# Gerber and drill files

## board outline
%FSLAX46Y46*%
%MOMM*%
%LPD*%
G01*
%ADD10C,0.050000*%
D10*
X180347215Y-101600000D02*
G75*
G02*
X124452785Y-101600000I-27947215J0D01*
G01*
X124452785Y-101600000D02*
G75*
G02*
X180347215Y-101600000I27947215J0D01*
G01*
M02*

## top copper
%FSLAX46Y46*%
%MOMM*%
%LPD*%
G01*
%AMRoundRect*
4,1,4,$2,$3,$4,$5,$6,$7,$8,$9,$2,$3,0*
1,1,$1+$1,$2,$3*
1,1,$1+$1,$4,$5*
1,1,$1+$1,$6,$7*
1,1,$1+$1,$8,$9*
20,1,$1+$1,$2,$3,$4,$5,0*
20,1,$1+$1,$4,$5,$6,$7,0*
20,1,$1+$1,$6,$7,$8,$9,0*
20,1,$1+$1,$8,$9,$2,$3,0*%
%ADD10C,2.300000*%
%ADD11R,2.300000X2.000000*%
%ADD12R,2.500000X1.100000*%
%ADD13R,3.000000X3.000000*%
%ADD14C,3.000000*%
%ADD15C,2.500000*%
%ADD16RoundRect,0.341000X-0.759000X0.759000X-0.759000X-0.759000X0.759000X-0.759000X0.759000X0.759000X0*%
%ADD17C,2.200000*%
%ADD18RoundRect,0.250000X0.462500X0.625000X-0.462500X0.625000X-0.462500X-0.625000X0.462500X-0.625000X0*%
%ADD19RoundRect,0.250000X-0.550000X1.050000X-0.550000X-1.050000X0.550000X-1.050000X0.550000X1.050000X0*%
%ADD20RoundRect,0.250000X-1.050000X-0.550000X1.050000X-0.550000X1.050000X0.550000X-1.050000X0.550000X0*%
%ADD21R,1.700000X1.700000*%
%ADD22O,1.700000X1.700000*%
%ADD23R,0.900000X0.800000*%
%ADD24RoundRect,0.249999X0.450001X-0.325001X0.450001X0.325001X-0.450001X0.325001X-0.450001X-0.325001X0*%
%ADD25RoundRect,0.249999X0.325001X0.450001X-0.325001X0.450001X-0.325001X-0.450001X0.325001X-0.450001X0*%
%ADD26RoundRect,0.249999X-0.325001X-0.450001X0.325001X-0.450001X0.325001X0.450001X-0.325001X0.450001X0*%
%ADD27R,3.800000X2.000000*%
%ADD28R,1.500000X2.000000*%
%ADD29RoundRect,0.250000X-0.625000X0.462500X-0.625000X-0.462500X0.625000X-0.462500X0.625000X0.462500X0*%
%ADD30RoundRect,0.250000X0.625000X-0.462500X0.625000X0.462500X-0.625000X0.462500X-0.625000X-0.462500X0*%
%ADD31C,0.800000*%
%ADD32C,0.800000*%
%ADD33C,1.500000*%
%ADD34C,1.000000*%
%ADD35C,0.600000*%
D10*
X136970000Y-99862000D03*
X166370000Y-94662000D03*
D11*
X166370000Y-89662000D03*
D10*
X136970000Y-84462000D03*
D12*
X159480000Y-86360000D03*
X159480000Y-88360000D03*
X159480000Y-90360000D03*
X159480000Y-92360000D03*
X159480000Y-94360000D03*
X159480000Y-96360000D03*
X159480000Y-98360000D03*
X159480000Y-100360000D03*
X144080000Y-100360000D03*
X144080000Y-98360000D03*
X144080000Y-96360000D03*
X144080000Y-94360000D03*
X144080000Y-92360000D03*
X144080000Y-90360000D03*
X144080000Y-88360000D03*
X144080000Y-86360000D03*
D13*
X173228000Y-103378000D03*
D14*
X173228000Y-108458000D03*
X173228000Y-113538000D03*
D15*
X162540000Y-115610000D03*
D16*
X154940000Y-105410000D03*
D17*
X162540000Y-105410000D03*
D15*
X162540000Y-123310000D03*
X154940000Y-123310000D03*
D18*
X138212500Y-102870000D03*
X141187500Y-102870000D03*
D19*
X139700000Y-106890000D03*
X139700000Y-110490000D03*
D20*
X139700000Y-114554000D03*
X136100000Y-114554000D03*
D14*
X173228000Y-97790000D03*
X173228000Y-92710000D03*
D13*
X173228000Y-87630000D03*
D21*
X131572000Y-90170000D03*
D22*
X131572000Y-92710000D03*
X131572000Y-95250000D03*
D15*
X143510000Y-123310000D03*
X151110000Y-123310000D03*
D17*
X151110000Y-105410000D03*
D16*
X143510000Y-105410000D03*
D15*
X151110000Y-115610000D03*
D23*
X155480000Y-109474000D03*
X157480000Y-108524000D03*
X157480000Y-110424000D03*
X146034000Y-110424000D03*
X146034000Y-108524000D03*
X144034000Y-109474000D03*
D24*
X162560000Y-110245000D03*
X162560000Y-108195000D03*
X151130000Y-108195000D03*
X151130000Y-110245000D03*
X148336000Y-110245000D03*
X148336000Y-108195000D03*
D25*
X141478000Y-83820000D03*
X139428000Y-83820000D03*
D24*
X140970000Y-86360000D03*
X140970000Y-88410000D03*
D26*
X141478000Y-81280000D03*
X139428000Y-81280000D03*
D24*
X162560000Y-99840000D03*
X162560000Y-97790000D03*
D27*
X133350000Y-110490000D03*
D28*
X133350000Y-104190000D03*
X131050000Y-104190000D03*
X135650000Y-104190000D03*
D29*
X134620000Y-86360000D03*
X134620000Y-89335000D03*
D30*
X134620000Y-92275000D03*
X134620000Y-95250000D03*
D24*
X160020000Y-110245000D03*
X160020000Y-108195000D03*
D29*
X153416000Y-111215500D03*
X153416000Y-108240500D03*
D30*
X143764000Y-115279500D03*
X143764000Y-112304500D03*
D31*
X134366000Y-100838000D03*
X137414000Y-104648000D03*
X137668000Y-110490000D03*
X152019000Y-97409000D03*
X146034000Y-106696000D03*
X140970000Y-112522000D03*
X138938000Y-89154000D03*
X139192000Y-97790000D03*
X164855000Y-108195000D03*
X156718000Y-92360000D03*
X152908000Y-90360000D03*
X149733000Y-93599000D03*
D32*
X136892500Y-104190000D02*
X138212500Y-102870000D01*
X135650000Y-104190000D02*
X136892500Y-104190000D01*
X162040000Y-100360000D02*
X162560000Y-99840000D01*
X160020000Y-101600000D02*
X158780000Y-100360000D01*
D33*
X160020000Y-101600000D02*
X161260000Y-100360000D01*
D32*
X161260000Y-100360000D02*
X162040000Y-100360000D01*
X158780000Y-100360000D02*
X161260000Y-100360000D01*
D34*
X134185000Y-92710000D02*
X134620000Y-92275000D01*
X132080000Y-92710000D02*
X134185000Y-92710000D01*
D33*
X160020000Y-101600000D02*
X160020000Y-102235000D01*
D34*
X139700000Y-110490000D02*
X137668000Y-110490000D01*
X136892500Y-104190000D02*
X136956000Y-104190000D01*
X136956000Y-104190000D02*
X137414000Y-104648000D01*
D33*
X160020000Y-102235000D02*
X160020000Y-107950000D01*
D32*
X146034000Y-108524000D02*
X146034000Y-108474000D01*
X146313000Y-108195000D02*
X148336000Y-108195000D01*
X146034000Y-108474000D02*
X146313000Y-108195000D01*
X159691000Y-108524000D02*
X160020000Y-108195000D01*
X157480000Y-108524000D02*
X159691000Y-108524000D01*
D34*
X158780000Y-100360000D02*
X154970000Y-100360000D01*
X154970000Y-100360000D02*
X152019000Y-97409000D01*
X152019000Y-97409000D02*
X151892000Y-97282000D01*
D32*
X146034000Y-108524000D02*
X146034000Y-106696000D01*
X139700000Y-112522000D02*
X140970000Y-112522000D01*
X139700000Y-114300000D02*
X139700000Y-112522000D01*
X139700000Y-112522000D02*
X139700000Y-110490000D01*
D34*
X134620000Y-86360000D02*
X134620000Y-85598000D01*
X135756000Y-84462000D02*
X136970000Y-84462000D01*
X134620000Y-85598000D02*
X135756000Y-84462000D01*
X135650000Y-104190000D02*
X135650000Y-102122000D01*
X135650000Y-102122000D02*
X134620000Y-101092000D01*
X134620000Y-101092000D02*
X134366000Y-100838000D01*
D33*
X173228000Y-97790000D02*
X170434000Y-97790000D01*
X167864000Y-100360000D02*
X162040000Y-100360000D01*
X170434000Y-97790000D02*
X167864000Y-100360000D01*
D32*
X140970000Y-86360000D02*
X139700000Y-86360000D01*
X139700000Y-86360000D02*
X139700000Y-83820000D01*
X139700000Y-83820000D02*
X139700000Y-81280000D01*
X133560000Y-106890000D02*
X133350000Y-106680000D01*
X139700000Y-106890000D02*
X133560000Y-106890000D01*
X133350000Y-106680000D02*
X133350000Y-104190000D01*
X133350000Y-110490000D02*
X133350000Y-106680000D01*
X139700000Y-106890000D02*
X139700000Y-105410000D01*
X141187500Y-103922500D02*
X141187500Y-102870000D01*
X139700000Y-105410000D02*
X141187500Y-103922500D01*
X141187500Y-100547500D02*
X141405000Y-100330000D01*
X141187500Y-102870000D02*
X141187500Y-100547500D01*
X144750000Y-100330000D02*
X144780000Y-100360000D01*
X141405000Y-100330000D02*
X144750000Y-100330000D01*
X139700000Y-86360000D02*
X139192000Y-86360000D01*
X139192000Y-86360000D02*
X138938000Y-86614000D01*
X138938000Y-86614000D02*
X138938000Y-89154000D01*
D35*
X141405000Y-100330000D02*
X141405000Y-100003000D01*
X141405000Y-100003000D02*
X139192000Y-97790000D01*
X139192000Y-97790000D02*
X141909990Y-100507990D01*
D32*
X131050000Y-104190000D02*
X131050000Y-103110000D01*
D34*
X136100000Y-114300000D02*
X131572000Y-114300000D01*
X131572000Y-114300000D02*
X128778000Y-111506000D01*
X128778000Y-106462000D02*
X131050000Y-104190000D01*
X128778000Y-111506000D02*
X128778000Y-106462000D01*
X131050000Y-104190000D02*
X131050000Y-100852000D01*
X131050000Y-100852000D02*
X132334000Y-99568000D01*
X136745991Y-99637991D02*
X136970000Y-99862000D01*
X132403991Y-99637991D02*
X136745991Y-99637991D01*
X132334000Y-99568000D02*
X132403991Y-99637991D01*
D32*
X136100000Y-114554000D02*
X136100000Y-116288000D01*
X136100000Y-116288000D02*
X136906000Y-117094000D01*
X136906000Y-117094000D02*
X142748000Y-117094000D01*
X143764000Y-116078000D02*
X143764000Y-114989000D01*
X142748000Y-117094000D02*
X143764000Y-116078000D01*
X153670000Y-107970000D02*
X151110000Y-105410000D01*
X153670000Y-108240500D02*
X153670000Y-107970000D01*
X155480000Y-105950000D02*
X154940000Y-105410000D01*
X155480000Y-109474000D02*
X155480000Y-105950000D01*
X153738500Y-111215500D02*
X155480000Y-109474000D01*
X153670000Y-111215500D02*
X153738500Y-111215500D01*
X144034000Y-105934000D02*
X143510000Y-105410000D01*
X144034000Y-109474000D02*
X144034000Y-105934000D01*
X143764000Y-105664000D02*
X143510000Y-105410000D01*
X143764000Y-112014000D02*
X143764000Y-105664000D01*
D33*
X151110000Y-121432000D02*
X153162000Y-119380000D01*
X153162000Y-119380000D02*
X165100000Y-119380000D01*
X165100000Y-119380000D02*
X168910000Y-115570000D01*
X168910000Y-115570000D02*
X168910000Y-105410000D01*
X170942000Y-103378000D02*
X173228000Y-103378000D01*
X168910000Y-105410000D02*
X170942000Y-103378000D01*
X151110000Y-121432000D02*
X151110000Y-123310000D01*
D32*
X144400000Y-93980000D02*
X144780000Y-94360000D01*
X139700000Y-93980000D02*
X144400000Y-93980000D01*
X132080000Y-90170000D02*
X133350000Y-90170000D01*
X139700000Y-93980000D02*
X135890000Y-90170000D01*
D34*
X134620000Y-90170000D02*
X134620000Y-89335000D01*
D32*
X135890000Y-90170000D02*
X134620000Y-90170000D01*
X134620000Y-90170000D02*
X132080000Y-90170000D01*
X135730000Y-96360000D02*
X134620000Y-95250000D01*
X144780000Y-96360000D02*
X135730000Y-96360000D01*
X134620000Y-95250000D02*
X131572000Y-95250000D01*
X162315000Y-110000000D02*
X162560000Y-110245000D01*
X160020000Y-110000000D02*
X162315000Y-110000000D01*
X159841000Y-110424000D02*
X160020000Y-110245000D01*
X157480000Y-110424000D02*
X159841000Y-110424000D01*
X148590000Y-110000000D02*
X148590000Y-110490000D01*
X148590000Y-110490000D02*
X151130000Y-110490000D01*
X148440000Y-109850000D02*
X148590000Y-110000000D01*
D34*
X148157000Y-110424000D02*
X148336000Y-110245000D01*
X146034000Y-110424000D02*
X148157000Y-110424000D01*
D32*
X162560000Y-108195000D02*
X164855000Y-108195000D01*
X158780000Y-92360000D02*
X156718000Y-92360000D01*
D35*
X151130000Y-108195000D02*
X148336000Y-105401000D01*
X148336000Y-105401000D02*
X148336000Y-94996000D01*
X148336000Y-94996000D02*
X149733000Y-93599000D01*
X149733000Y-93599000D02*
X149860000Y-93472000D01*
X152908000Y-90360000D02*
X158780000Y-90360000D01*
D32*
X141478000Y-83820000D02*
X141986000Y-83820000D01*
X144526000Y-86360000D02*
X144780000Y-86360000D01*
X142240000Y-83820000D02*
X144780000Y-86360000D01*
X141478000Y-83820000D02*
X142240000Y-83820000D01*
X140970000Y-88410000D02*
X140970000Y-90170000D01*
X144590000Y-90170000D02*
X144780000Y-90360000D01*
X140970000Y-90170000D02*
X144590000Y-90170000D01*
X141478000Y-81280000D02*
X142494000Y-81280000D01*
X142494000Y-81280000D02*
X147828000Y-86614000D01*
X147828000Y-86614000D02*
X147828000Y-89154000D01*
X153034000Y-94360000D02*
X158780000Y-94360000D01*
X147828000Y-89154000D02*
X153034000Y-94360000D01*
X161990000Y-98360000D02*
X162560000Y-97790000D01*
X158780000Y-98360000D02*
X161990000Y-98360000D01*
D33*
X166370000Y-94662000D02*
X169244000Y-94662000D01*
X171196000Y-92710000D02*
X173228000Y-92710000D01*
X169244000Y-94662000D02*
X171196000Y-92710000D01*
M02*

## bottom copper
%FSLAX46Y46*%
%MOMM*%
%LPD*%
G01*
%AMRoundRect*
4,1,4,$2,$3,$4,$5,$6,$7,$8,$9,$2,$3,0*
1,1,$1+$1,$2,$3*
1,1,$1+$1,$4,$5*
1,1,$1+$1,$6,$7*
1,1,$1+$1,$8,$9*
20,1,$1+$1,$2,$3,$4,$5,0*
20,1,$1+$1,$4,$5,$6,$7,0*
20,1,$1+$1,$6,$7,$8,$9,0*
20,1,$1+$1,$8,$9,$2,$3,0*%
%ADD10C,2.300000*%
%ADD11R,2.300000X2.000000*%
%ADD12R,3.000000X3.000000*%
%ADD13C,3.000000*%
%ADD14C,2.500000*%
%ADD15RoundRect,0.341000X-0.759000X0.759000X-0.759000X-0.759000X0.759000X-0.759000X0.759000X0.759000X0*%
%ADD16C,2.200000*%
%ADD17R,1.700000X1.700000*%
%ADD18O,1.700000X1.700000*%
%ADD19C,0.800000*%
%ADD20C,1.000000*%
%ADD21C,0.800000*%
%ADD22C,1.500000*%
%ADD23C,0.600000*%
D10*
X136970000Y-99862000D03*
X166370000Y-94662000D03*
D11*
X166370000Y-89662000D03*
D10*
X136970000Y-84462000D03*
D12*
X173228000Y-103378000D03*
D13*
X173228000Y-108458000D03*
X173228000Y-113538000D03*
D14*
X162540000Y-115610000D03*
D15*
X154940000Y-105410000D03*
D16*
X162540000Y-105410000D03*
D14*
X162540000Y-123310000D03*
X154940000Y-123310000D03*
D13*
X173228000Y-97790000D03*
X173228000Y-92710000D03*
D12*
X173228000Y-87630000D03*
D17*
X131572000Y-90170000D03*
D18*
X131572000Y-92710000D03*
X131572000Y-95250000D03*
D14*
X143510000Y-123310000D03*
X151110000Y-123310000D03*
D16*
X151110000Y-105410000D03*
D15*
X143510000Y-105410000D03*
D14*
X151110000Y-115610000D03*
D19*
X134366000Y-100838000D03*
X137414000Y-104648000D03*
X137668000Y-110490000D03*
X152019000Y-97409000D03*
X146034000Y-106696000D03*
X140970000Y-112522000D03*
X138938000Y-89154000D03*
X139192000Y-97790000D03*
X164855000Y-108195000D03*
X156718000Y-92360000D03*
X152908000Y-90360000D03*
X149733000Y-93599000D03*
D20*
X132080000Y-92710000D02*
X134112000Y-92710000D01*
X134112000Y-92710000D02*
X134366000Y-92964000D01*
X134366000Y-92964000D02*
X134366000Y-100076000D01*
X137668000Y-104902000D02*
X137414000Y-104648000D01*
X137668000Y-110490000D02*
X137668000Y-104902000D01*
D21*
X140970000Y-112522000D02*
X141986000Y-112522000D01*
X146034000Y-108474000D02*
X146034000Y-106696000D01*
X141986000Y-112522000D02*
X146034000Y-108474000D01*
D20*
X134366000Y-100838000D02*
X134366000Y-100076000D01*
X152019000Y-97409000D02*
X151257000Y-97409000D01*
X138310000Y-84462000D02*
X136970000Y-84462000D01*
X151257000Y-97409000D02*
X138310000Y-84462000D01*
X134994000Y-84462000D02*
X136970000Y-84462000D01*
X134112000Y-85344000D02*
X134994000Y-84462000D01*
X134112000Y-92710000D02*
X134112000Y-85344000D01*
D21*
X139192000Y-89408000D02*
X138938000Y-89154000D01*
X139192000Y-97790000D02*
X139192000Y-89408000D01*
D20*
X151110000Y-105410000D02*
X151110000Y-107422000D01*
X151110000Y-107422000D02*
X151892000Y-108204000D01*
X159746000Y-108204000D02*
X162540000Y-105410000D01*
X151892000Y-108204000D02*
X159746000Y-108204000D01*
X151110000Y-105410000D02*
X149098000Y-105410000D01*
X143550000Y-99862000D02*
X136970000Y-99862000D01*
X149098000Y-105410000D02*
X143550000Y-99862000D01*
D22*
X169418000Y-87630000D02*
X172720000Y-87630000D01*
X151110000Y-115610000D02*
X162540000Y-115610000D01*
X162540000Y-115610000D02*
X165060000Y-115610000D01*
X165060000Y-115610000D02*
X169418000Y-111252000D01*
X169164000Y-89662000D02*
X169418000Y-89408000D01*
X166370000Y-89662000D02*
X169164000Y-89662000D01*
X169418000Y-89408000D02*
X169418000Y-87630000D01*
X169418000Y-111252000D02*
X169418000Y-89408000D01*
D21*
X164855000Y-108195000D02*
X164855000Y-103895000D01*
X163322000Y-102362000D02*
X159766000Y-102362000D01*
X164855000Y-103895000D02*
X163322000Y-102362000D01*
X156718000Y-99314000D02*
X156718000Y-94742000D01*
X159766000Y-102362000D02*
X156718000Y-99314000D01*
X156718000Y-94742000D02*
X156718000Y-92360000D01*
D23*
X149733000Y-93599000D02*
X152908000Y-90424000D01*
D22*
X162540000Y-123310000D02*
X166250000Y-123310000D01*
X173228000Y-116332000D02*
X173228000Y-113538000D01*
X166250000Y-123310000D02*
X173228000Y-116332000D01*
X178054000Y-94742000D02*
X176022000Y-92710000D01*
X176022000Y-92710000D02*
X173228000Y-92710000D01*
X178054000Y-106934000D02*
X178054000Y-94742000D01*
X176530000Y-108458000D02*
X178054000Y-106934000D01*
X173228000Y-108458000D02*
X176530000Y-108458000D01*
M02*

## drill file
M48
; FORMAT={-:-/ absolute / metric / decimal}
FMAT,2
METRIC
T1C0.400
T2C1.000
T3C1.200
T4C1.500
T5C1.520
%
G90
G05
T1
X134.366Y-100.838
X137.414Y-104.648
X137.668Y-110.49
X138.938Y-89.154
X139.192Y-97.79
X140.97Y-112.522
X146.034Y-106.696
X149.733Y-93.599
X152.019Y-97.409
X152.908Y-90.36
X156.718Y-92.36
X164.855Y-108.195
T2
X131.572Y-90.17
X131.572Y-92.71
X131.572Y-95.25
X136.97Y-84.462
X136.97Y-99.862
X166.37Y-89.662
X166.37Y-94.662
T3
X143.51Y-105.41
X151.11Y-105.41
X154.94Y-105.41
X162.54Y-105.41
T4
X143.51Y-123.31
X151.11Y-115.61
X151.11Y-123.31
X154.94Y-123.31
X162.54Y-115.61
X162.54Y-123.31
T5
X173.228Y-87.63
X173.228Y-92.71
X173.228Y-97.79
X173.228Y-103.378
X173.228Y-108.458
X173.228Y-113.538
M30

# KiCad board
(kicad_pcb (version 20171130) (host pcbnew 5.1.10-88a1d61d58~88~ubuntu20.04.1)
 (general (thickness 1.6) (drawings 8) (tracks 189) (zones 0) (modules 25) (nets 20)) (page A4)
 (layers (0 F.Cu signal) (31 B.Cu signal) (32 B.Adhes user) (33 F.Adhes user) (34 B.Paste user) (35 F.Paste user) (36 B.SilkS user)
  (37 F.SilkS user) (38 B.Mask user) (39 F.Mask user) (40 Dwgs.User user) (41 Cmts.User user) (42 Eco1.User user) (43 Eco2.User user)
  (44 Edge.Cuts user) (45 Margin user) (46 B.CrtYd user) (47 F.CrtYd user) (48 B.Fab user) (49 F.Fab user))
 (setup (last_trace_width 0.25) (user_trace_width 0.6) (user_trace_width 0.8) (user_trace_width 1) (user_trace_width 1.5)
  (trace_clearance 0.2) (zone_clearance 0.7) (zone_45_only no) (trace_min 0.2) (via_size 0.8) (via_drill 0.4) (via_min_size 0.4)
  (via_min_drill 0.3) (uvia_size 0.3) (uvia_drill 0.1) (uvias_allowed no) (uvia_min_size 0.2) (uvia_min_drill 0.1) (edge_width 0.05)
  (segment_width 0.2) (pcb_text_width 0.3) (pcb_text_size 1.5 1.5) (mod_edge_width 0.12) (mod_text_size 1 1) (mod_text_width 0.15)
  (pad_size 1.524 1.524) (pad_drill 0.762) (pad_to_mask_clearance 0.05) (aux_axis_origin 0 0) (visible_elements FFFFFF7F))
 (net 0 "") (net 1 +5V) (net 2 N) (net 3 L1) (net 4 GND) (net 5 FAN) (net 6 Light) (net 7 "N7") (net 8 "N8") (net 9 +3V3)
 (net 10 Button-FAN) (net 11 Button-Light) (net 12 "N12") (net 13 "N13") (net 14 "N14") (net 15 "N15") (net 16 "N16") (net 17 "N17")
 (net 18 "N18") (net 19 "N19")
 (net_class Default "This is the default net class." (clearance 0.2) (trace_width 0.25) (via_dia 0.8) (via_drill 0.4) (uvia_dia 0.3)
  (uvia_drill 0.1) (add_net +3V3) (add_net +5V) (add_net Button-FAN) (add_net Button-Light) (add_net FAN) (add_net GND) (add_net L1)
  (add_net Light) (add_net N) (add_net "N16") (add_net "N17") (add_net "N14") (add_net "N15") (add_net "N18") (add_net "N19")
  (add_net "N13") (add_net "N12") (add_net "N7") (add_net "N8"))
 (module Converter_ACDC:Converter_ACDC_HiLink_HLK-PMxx (layer B.Cu) (at 166.37 89.662 180)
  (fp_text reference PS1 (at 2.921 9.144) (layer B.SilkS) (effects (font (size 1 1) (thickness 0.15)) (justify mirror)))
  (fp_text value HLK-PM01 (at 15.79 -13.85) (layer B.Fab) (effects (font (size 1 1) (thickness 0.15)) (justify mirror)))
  (pad 4 thru_hole circle (at 29.4 -10.2 180) (size 2.3 2.3) (drill 1) (layers *.Cu *.Mask) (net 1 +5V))
  (pad 2 thru_hole circle (at 0 -5 180) (size 2.3 2.3) (drill 1) (layers *.Cu *.Mask) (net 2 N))
  (pad 1 thru_hole rect (at 0 0 180) (size 2.3 2) (drill 1) (layers *.Cu *.Mask) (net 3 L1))
  (pad 3 thru_hole circle (at 29.4 5.2 180) (size 2.3 2.3) (drill 1) (layers *.Cu *.Mask) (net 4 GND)))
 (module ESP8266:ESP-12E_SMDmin (layer F.Cu) (at 144.78 86.36)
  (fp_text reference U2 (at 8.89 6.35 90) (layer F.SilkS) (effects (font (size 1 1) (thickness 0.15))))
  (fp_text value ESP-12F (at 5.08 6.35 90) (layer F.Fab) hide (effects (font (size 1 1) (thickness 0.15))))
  (pad 16 smd rect (at 14 0) (size 2.5 1.1) (drill (offset 0.7 0)) (layers F.Cu F.Paste F.Mask))
  (pad 15 smd rect (at 14 2) (size 2.5 1.1) (drill (offset 0.7 0)) (layers F.Cu F.Paste F.Mask))
  (pad 14 smd rect (at 14 4) (size 2.5 1.1) (drill (offset 0.7 0)) (layers F.Cu F.Paste F.Mask) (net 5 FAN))
  (pad 13 smd rect (at 14 6) (size 2.5 1.1) (drill (offset 0.7 0)) (layers F.Cu F.Paste F.Mask) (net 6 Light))
  (pad 12 smd rect (at 14 8) (size 2.5 1.1) (drill (offset 0.7 0)) (layers F.Cu F.Paste F.Mask) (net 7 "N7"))
  (pad 11 smd rect (at 14 10) (size 2.5 1.1) (drill (offset 0.7 0)) (layers F.Cu F.Paste F.Mask))
  (pad 10 smd rect (at 14 12) (size 2.5 1.1) (drill (offset 0.7 0)) (layers F.Cu F.Paste F.Mask) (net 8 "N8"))
  (pad 9 smd rect (at 14 14) (size 2.5 1.1) (drill (offset 0.7 0)) (layers F.Cu F.Paste F.Mask) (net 4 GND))
  (pad 8 smd rect (at 0 14) (size 2.5 1.1) (drill (offset -0.7 0)) (layers F.Cu F.Paste F.Mask) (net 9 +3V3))
  (pad 7 smd rect (at 0 12) (size 2.5 1.1) (drill (offset -0.7 0)) (layers F.Cu F.Paste F.Mask))
  (pad 6 smd rect (at 0 10) (size 2.5 1.1) (drill (offset -0.7 0)) (layers F.Cu F.Paste F.Mask) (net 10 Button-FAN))
  (pad 5 smd rect (at 0 8) (size 2.5 1.1) (drill (offset -0.7 0)) (layers F.Cu F.Paste F.Mask) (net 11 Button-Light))
  (pad 4 smd rect (at 0 6) (size 2.5 1.1) (drill (offset -0.7 0)) (layers F.Cu F.Paste F.Mask))
  (pad 3 smd rect (at 0 4) (size 2.5 1.1) (drill (offset -0.7 0)) (layers F.Cu F.Paste F.Mask) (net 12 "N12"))
  (pad 2 smd rect (at 0 2) (size 2.5 1.1) (drill (offset -0.7 0)) (layers F.Cu F.Paste F.Mask))
  (pad 1 smd rect (at 0 0) (size 2.5 1.1) (drill (offset -0.7 0)) (layers F.Cu F.Paste F.Mask) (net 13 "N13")))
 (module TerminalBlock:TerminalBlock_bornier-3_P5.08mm (layer B.Cu) (at 173.228 103.378 270)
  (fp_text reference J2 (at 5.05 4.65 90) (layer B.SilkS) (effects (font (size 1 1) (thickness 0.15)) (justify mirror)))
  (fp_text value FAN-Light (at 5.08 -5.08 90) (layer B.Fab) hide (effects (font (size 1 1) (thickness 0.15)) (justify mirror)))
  (pad 1 thru_hole rect (at 0 0 270) (size 3 3) (drill 1.52) (layers *.Cu *.Mask) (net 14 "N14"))
  (pad 2 thru_hole circle (at 5.08 0 270) (size 3 3) (drill 1.52) (layers *.Cu *.Mask) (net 2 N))
  (pad 3 thru_hole circle (at 10.16 0 270) (size 3 3) (drill 1.52) (layers *.Cu *.Mask) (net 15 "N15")))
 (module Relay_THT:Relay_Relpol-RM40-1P (layer B.Cu) (at 154.94 105.41 270)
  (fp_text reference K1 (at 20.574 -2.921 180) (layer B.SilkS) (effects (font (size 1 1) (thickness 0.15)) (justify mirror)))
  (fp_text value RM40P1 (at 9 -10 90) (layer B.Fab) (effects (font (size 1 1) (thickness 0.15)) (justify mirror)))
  (pad 11 thru_hole circle (at 10.2 -7.6 270) (size 2.5 2.5) (drill 1.5) (layers *.Cu *.Mask) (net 3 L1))
  (pad A2 thru_hole roundrect (at 0 0 270) (size 2.2 2.2) (drill 1.2) (layers *.Cu *.Mask) (roundrect_rratio 0.155) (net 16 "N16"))
  (pad A1 thru_hole circle (at 0 -7.6 270) (size 2.2 2.2) (drill 1.2) (layers *.Cu *.Mask) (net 1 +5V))
  (pad 14 thru_hole circle (at 17.9 -7.6 270) (size 2.5 2.5) (drill 1.5) (layers *.Cu *.Mask) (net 15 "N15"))
  (pad 12 thru_hole circle (at 17.9 0 270) (size 2.5 2.5) (drill 1.5) (layers *.Cu *.Mask)))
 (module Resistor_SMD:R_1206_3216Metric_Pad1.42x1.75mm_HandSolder (layer F.Cu) (at 139.7 102.87 180)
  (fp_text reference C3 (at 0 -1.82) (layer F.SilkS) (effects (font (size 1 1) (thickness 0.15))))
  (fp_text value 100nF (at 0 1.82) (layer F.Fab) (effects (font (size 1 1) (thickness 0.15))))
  (pad 2 smd roundrect (at 1.4875 0 180) (size 1.425 1.75) (layers F.Cu F.Paste F.Mask) (roundrect_rratio 0.1754385964912281) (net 4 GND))
  (pad 1 smd roundrect (at -1.4875 0 180) (size 1.425 1.75) (layers F.Cu F.Paste F.Mask) (roundrect_rratio 0.1754385964912281) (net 9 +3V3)))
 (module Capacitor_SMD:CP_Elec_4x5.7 (layer F.Cu) (at 139.7 108.69 270)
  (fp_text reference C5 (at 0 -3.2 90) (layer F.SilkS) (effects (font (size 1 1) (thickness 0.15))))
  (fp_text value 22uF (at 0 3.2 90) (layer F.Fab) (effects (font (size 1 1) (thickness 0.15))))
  (pad 1 smd roundrect (at -1.8 0 270) (size 2.6 1.6) (layers F.Cu F.Paste F.Mask) (roundrect_rratio 0.15625) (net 9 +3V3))
  (pad 2 smd roundrect (at 1.8 0 270) (size 2.6 1.6) (layers F.Cu F.Paste F.Mask) (roundrect_rratio 0.15625) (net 4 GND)))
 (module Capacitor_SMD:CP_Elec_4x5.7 (layer F.Cu) (at 137.9 114.554)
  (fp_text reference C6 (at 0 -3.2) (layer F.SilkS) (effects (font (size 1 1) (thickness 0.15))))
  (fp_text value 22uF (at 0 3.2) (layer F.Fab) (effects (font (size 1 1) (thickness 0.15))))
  (pad 2 smd roundrect (at 1.8 0) (size 2.6 1.6) (layers F.Cu F.Paste F.Mask) (roundrect_rratio 0.15625) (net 4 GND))
  (pad 1 smd roundrect (at -1.8 0) (size 2.6 1.6) (layers F.Cu F.Paste F.Mask) (roundrect_rratio 0.15625) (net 1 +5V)))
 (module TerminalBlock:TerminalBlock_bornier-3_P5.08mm (layer B.Cu) (at 173.228 87.63 270)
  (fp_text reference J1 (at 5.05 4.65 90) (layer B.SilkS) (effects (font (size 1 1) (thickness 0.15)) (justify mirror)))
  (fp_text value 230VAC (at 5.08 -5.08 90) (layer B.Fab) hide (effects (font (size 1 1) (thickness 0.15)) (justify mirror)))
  (pad 3 thru_hole circle (at 10.16 0 270) (size 3 3) (drill 1.52) (layers *.Cu *.Mask) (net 4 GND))
  (pad 2 thru_hole circle (at 5.08 0 270) (size 3 3) (drill 1.52) (layers *.Cu *.Mask) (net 2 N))
  (pad 1 thru_hole rect (at 0 0 270) (size 3 3) (drill 1.52) (layers *.Cu *.Mask) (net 3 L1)))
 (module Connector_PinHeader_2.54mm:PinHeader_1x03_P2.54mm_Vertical (layer F.Cu) (at 131.572 90.17)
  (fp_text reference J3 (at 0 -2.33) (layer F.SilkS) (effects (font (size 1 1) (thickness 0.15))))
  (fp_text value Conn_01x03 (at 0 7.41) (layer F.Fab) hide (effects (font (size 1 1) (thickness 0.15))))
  (pad 1 thru_hole rect (at 0 0) (size 1.7 1.7) (drill 1) (layers *.Cu *.Mask) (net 11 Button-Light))
  (pad 2 thru_hole oval (at 0 2.54) (size 1.7 1.7) (drill 1) (layers *.Cu *.Mask) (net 4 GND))
  (pad 3 thru_hole oval (at 0 5.08) (size 1.7 1.7) (drill 1) (layers *.Cu *.Mask) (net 10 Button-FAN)))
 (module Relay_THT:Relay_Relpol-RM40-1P (layer B.Cu) (at 143.51 105.41 270)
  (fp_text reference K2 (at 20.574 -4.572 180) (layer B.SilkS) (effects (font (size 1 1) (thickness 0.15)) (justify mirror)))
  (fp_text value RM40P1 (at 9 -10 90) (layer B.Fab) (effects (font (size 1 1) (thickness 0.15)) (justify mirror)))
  (pad 12 thru_hole circle (at 17.9 0 270) (size 2.5 2.5) (drill 1.5) (layers *.Cu *.Mask))
  (pad 14 thru_hole circle (at 17.9 -7.6 270) (size 2.5 2.5) (drill 1.5) (layers *.Cu *.Mask) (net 14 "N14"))
  (pad A1 thru_hole circle (at 0 -7.6 270) (size 2.2 2.2) (drill 1.2) (layers *.Cu *.Mask) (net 1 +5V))
  (pad A2 thru_hole roundrect (at 0 0 270) (size 2.2 2.2) (drill 1.2) (layers *.Cu *.Mask) (roundrect_rratio 0.155) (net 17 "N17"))
  (pad 11 thru_hole circle (at 10.2 -7.6 270) (size 2.5 2.5) (drill 1.5) (layers *.Cu *.Mask) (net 3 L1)))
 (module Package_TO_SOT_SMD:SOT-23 (layer F.Cu) (at 156.48 109.474 180)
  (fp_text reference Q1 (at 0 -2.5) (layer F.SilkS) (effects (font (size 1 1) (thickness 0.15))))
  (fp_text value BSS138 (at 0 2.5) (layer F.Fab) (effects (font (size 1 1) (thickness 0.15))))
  (pad 3 smd rect (at 1 0 180) (size 0.9 0.8) (layers F.Cu F.Paste F.Mask) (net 16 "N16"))
  (pad 2 smd rect (at -1 0.95 180) (size 0.9 0.8) (layers F.Cu F.Paste F.Mask) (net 4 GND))
  (pad 1 smd rect (at -1 -0.95 180) (size 0.9 0.8) (layers F.Cu F.Paste F.Mask) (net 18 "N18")))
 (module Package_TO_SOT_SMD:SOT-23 (layer F.Cu) (at 145.034 109.474 180)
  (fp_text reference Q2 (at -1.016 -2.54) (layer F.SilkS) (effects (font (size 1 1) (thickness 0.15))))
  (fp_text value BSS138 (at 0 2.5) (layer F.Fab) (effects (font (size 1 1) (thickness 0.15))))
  (pad 1 smd rect (at -1 -0.95 180) (size 0.9 0.8) (layers F.Cu F.Paste F.Mask) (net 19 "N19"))
  (pad 2 smd rect (at -1 0.95 180) (size 0.9 0.8) (layers F.Cu F.Paste F.Mask) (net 4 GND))
  (pad 3 smd rect (at 1 0 180) (size 0.9 0.8) (layers F.Cu F.Paste F.Mask) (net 17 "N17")))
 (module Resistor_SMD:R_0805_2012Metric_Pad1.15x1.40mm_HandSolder (layer F.Cu) (at 162.56 109.22 90)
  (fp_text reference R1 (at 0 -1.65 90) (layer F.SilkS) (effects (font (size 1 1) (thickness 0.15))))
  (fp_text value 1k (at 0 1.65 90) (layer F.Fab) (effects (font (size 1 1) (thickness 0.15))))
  (pad 1 smd roundrect (at -1.025 0 90) (size 1.15 1.4) (layers F.Cu F.Paste F.Mask) (roundrect_rratio 0.2173904347826087) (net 18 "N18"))
  (pad 2 smd roundrect (at 1.025 0 90) (size 1.15 1.4) (layers F.Cu F.Paste F.Mask) (roundrect_rratio 0.2173904347826087) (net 6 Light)))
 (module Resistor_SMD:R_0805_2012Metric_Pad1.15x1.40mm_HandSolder (layer F.Cu) (at 151.13 109.22 90)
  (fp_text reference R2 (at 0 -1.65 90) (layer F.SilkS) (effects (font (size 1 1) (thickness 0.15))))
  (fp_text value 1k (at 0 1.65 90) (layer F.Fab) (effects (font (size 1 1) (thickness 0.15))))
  (pad 2 smd roundrect (at 1.025 0 90) (size 1.15 1.4) (layers F.Cu F.Paste F.Mask) (roundrect_rratio 0.2173904347826087) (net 5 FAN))
  (pad 1 smd roundrect (at -1.025 0 90) (size 1.15 1.4) (layers F.Cu F.Paste F.Mask) (roundrect_rratio 0.2173904347826087) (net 19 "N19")))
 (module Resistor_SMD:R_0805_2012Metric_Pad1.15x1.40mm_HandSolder (layer F.Cu) (at 148.336 109.22 90)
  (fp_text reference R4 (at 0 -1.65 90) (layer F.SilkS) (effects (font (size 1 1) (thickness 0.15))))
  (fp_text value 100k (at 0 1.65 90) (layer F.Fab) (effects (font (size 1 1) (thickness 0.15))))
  (pad 1 smd roundrect (at -1.025 0 90) (size 1.15 1.4) (layers F.Cu F.Paste F.Mask) (roundrect_rratio 0.2173904347826087) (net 19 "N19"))
  (pad 2 smd roundrect (at 1.025 0 90) (size 1.15 1.4) (layers F.Cu F.Paste F.Mask) (roundrect_rratio 0.2173904347826087) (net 4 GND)))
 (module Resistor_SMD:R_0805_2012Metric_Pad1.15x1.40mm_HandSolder (layer F.Cu) (at 140.453 83.82 180)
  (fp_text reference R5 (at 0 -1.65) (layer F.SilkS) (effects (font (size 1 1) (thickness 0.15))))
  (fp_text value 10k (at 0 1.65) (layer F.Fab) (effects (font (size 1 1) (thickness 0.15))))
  (pad 1 smd roundrect (at -1.025 0 180) (size 1.15 1.4) (layers F.Cu F.Paste F.Mask) (roundrect_rratio 0.2173904347826087) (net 13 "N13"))
  (pad 2 smd roundrect (at 1.025 0 180) (size 1.15 1.4) (layers F.Cu F.Paste F.Mask) (roundrect_rratio 0.2173904347826087) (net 9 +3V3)))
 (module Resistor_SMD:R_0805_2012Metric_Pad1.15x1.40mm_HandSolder (layer F.Cu) (at 140.97 87.385 90)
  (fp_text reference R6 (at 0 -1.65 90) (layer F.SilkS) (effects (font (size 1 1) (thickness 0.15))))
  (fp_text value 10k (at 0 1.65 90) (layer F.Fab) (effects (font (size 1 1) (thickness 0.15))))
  (pad 2 smd roundrect (at 1.025 0 90) (size 1.15 1.4) (layers F.Cu F.Paste F.Mask) (roundrect_rratio 0.2173904347826087) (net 9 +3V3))
  (pad 1 smd roundrect (at -1.025 0 90) (size 1.15 1.4) (layers F.Cu F.Paste F.Mask) (roundrect_rratio 0.2173904347826087) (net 12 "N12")))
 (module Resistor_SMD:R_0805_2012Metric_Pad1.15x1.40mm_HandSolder (layer F.Cu) (at 140.453 81.28)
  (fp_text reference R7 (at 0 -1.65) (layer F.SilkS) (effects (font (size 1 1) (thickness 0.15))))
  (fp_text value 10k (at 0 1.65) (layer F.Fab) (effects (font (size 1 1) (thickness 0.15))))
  (pad 2 smd roundrect (at 1.025 0) (size 1.15 1.4) (layers F.Cu F.Paste F.Mask) (roundrect_rratio 0.2173904347826087) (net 7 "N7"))
  (pad 1 smd roundrect (at -1.025 0) (size 1.15 1.4) (layers F.Cu F.Paste F.Mask) (roundrect_rratio 0.2173904347826087) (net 9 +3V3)))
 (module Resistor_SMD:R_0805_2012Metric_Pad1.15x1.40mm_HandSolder (layer F.Cu) (at 162.56 98.815 90)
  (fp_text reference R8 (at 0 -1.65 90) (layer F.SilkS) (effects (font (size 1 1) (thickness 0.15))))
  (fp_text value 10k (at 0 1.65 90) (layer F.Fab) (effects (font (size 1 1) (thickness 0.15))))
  (pad 1 smd roundrect (at -1.025 0 90) (size 1.15 1.4) (layers F.Cu F.Paste F.Mask) (roundrect_rratio 0.2173904347826087) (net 4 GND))
  (pad 2 smd roundrect (at 1.025 0 90) (size 1.15 1.4) (layers F.Cu F.Paste F.Mask) (roundrect_rratio 0.2173904347826087) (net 8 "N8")))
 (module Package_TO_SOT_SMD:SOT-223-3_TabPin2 (layer F.Cu) (at 133.35 107.34 270)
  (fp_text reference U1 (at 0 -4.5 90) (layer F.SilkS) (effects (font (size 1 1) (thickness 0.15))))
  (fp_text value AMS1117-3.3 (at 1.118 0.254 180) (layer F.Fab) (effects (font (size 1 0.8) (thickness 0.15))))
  (pad 2 smd rect (at 3.15 0 270) (size 2 3.8) (layers F.Cu F.Paste F.Mask) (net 9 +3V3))
  (pad 2 smd rect (at -3.15 0 270) (size 2 1.5) (layers F.Cu F.Paste F.Mask) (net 9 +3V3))
  (pad 3 smd rect (at -3.15 2.3 270) (size 2 1.5) (layers F.Cu F.Paste F.Mask) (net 1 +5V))
  (pad 1 smd rect (at -3.15 -2.3 270) (size 2 1.5) (layers F.Cu F.Paste F.Mask) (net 4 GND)))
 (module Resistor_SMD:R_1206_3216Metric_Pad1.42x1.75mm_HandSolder (layer F.Cu) (at 134.62 87.8475 270)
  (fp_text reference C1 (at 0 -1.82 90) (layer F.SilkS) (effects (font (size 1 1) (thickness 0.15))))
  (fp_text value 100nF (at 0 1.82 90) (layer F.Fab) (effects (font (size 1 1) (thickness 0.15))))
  (pad 1 smd roundrect (at -1.4875 0 270) (size 1.425 1.75) (layers F.Cu F.Paste F.Mask) (roundrect_rratio 0.1754385964912281) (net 4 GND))
  (pad 2 smd roundrect (at 1.4875 0 270) (size 1.425 1.75) (layers F.Cu F.Paste F.Mask) (roundrect_rratio 0.1754385964912281)
   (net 11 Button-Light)))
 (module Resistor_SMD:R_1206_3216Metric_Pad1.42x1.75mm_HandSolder (layer F.Cu) (at 134.62 93.7625 90)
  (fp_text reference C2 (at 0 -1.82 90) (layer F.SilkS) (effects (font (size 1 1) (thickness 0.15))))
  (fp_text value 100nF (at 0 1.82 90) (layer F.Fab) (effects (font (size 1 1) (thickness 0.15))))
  (pad 2 smd roundrect (at 1.4875 0 90) (size 1.425 1.75) (layers F.Cu F.Paste F.Mask) (roundrect_rratio 0.1754385964912281) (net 4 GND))
  (pad 1 smd roundrect (at -1.4875 0 90) (size 1.425 1.75) (layers F.Cu F.Paste F.Mask) (roundrect_rratio 0.1754385964912281)
   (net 10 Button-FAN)))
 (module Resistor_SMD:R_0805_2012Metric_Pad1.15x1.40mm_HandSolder (layer F.Cu) (at 160.02 109.22 90)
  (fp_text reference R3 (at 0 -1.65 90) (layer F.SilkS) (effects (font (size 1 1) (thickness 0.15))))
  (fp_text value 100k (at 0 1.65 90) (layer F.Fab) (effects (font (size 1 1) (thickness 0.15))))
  (pad 1 smd roundrect (at -1.025 0 90) (size 1.15 1.4) (layers F.Cu F.Paste F.Mask) (roundrect_rratio 0.2173904347826087) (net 18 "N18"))
  (pad 2 smd roundrect (at 1.025 0 90) (size 1.15 1.4) (layers F.Cu F.Paste F.Mask) (roundrect_rratio 0.2173904347826087) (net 4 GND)))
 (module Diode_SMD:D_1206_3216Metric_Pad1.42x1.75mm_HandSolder (layer F.Cu) (at 153.416 109.728 270)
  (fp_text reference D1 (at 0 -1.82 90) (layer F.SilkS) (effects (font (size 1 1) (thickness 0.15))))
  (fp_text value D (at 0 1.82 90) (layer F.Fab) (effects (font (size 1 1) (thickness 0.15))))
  (pad 2 smd roundrect (at 1.4875 0 270) (size 1.425 1.75) (layers F.Cu F.Paste F.Mask) (roundrect_rratio 0.1754385964912281) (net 16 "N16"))
  (pad 1 smd roundrect (at -1.4875 0 270) (size 1.425 1.75) (layers F.Cu F.Paste F.Mask) (roundrect_rratio 0.1754385964912281) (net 1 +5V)))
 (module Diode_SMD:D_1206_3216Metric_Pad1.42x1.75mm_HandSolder (layer F.Cu) (at 143.764 113.792 90)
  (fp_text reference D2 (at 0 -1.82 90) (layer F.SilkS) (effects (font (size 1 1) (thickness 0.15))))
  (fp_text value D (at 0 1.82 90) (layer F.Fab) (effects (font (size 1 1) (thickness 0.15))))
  (pad 1 smd roundrect (at -1.4875 0 90) (size 1.425 1.75) (layers F.Cu F.Paste F.Mask) (roundrect_rratio 0.1754385964912281) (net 1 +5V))
  (pad 2 smd roundrect (at 1.4875 0 90) (size 1.425 1.75) (layers F.Cu F.Paste F.Mask) (roundrect_rratio 0.1754385964912281) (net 17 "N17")))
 (gr_circle (center 152.4 101.6) (end 153.035 73.66) (layer Edge.Cuts) (width 0.05))
 (segment (start 136.8925 104.19) (end 138.2125 102.87) (width 0.8) (layer F.Cu) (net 4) (status 20))
 (segment (start 135.65 104.19) (end 136.8925 104.19) (width 0.8) (layer F.Cu) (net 4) (status 10))
 (segment (start 162.04 100.36) (end 162.56 99.84) (width 0.8) (layer F.Cu) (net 4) (status 30))
 (segment (start 160.02 101.6) (end 158.78 100.36) (width 0.8) (layer F.Cu) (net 4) (status 20))
 (segment (start 160.02 101.6) (end 161.26 100.36) (width 1.5) (layer F.Cu) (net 4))
 (segment (start 161.26 100.36) (end 162.04 100.36) (width 0.8) (layer F.Cu) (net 4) (status 20))
 (segment (start 158.78 100.36) (end 161.26 100.36) (width 0.8) (layer F.Cu) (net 4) (status 10))
 (segment (start 134.185 92.71) (end 134.62 92.275) (width 1) (layer F.Cu) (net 4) (status 30))
 (segment (start 132.08 92.71) (end 134.185 92.71) (width 1) (layer F.Cu) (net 4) (status 30))
 (segment (start 160.02 101.6) (end 160.02 102.235) (width 1.5) (layer F.Cu) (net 4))
 (segment (start 132.08 92.71) (end 134.112 92.71) (width 1) (layer B.Cu) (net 4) (status 10))
 (segment (start 134.112 92.71) (end 134.366 92.964) (width 1) (layer B.Cu) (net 4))
 (segment (start 134.366 92.964) (end 134.366 100.076) (width 1) (layer B.Cu) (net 4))
 (via (at 134.366 100.838) (size 0.8) (drill 0.4) (layers F.Cu B.Cu) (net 4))
 (segment (start 139.7 110.49) (end 137.668 110.49) (width 1) (layer F.Cu) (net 4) (status 10))
 (segment (start 136.8925 104.19) (end 136.956 104.19) (width 1) (layer F.Cu) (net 4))
 (segment (start 136.956 104.19) (end 137.414 104.648) (width 1) (layer F.Cu) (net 4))
 (via (at 137.414 104.648) (size 0.8) (drill 0.4) (layers F.Cu B.Cu) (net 4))
 (via (at 137.668 110.49) (size 0.8) (drill 0.4) (layers F.Cu B.Cu) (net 4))
 (segment (start 137.668 104.902) (end 137.414 104.648) (width 1) (layer B.Cu) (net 4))
 (segment (start 137.668 110.49) (end 137.668 104.902) (width 1) (layer B.Cu) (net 4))
 (segment (start 160.02 102.235) (end 160.02 107.95) (width 1.5) (layer F.Cu) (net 4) (status 20))
 (segment (start 146.034 108.524) (end 146.034 108.474) (width 0.8) (layer F.Cu) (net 4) (status 30))
 (segment (start 146.313 108.195) (end 148.336 108.195) (width 0.8) (layer F.Cu) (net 4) (status 30))
 (segment (start 146.034 108.474) (end 146.313 108.195) (width 0.8) (layer F.Cu) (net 4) (status 30))
 (segment (start 159.691 108.524) (end 160.02 108.195) (width 0.8) (layer F.Cu) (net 4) (status 30))
 (segment (start 157.48 108.524) (end 159.691 108.524) (width 0.8) (layer F.Cu) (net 4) (status 30))
 (segment (start 158.78 100.36) (end 154.97 100.36) (width 1) (layer F.Cu) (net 4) (status 10))
 (segment (start 154.97 100.36) (end 152.019 97.409) (width 1) (layer F.Cu) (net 4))
 (segment (start 152.019 97.409) (end 151.892 97.282) (width 1) (layer F.Cu) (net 4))
 (via (at 152.019 97.409) (size 0.8) (drill 0.4) (layers F.Cu B.Cu) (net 4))
 (segment (start 146.034 108.524) (end 146.034 106.696) (width 0.8) (layer F.Cu) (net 4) (status 10))
 (via (at 146.034 106.696) (size 0.8) (drill 0.4) (layers F.Cu B.Cu) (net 4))
 (segment (start 139.7 112.522) (end 140.97 112.522) (width 0.8) (layer F.Cu) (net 4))
 (segment (start 139.7 114.3) (end 139.7 112.522) (width 0.8) (layer F.Cu) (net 4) (status 10))
 (segment (start 139.7 112.522) (end 139.7 110.49) (width 0.8) (layer F.Cu) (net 4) (status 20))
 (via (at 140.97 112.522) (size 0.8) (drill 0.4) (layers F.Cu B.Cu) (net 4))
 (segment (start 140.97 112.522) (end 141.986 112.522) (width 0.8) (layer B.Cu) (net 4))
 (segment (start 146.034 108.474) (end 146.034 106.696) (width 0.8) (layer B.Cu) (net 4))
 (segment (start 141.986 112.522) (end 146.034 108.474) (width 0.8) (layer B.Cu) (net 4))
 (segment (start 134.366 100.838) (end 134.366 100.076) (width 1) (layer B.Cu) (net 4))
 (segment (start 152.019 97.409) (end 151.257 97.409) (width 1) (layer B.Cu) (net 4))
 (segment (start 138.31 84.462) (end 136.97 84.462) (width 1) (layer B.Cu) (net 4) (status 20))
 (segment (start 151.257 97.409) (end 138.31 84.462) (width 1) (layer B.Cu) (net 4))
 (segment (start 134.62 86.36) (end 134.62 85.598) (width 1) (layer F.Cu) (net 4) (status 10))
 (segment (start 135.756 84.462) (end 136.97 84.462) (width 1) (layer F.Cu) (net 4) (status 20))
 (segment (start 134.62 85.598) (end 135.756 84.462) (width 1) (layer F.Cu) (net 4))
 (segment (start 135.65 104.19) (end 135.65 102.122) (width 1) (layer F.Cu) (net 4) (status 10))
 (segment (start 135.65 102.122) (end 134.62 101.092) (width 1) (layer F.Cu) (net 4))
 (segment (start 134.62 101.092) (end 134.366 100.838) (width 1) (layer F.Cu) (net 4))
 (segment (start 173.228 97.79) (end 170.434 97.79) (width 1.5) (layer F.Cu) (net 4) (status 10))
 (segment (start 167.864 100.36) (end 162.04 100.36) (width 1.5) (layer F.Cu) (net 4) (status 20))
 (segment (start 170.434 97.79) (end 167.864 100.36) (width 1.5) (layer F.Cu) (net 4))
 (segment (start 134.994 84.462) (end 136.97 84.462) (width 1) (layer B.Cu) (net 4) (status 20))
 (segment (start 134.112 85.344) (end 134.994 84.462) (width 1) (layer B.Cu) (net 4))
 (segment (start 134.112 92.71) (end 134.112 85.344) (width 1) (layer B.Cu) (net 4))
 (segment (start 140.97 86.36) (end 139.7 86.36) (width 0.8) (layer F.Cu) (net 9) (status 10))
 (segment (start 139.7 86.36) (end 139.7 83.82) (width 0.8) (layer F.Cu) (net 9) (status 20))
 (segment (start 139.7 83.82) (end 139.7 81.28) (width 0.8) (layer F.Cu) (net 9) (status 30))
 (segment (start 133.56 106.89) (end 133.35 106.68) (width 0.8) (layer F.Cu) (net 9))
 (segment (start 139.7 106.89) (end 133.56 106.89) (width 0.8) (layer F.Cu) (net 9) (status 10))
 (segment (start 133.35 106.68) (end 133.35 104.19) (width 0.8) (layer F.Cu) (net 9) (status 20))
 (segment (start 133.35 110.49) (end 133.35 106.68) (width 0.8) (layer F.Cu) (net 9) (status 10))
 (segment (start 139.7 106.89) (end 139.7 105.41) (width 0.8) (layer F.Cu) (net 9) (status 10))
 (segment (start 141.1875 103.9225) (end 141.1875 102.87) (width 0.8) (layer F.Cu) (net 9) (status 20))
 (segment (start 139.7 105.41) (end 141.1875 103.9225) (width 0.8) (layer F.Cu) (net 9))
 (segment (start 141.1875 100.5475) (end 141.405 100.33) (width 0.8) (layer F.Cu) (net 9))
 (segment (start 141.1875 102.87) (end 141.1875 100.5475) (width 0.8) (layer F.Cu) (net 9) (status 10))
 (segment (start 144.75 100.33) (end 144.78 100.36) (width 0.8) (layer F.Cu) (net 9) (status 30))
 (segment (start 141.405 100.33) (end 144.75 100.33) (width 0.8) (layer F.Cu) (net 9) (status 20))
 (segment (start 139.7 86.36) (end 139.192 86.36) (width 0.8) (layer F.Cu) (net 9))
 (segment (start 139.192 86.36) (end 138.938 86.614) (width 0.8) (layer F.Cu) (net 9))
 (segment (start 138.938 86.614) (end 138.938 89.154) (width 0.8) (layer F.Cu) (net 9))
 (via (at 138.938 89.154) (size 0.8) (drill 0.4) (layers F.Cu B.Cu) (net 9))
 (segment (start 141.405 100.33) (end 141.405 100.003) (width 0.6) (layer F.Cu) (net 9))
 (segment (start 141.405 100.003) (end 139.192 97.79) (width 0.6) (layer F.Cu) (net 9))
 (via (at 139.192 97.79) (size 0.8) (drill 0.4) (layers F.Cu B.Cu) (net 9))
 (segment (start 139.192 97.79) (end 141.90999 100.50799) (width 0.6) (layer F.Cu) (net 9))
 (segment (start 139.192 89.408) (end 138.938 89.154) (width 0.8) (layer B.Cu) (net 9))
 (segment (start 139.192 97.79) (end 139.192 89.408) (width 0.8) (layer B.Cu) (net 9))
 (segment (start 131.05 104.19) (end 131.05 103.11) (width 0.8) (layer F.Cu) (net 1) (status 10))
 (segment (start 151.11 105.41) (end 151.11 107.422) (width 1) (layer B.Cu) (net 1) (status 10))
 (segment (start 151.11 107.422) (end 151.892 108.204) (width 1) (layer B.Cu) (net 1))
 (segment (start 159.746 108.204) (end 162.54 105.41) (width 1) (layer B.Cu) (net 1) (status 20))
 (segment (start 151.892 108.204) (end 159.746 108.204) (width 1) (layer B.Cu) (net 1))
 (segment (start 136.1 114.3) (end 131.572 114.3) (width 1) (layer F.Cu) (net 1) (status 10))
 (segment (start 131.572 114.3) (end 128.778 111.506) (width 1) (layer F.Cu) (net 1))
 (segment (start 128.778 106.462) (end 131.05 104.19) (width 1) (layer F.Cu) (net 1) (status 20))
 (segment (start 128.778 111.506) (end 128.778 106.462) (width 1) (layer F.Cu) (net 1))
 (segment (start 151.11 105.41) (end 149.098 105.41) (width 1) (layer B.Cu) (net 1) (status 10))
 (segment (start 143.55 99.862) (end 136.97 99.862) (width 1) (layer B.Cu) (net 1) (status 20))
 (segment (start 149.098 105.41) (end 143.55 99.862) (width 1) (layer B.Cu) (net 1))
 (segment (start 131.05 104.19) (end 131.05 100.852) (width 1) (layer F.Cu) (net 1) (status 10))
 (segment (start 131.05 100.852) (end 132.334 99.568) (width 1) (layer F.Cu) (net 1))
 (segment (start 136.745991 99.637991) (end 136.97 99.862) (width 1) (layer F.Cu) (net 1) (status 30))
 (segment (start 132.403991 99.637991) (end 136.745991 99.637991) (width 1) (layer F.Cu) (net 1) (status 20))
 (segment (start 132.334 99.568) (end 132.403991 99.637991) (width 1) (layer F.Cu) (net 1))
 (segment (start 136.1 114.554) (end 136.1 116.288) (width 0.8) (layer F.Cu) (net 1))
 (segment (start 136.1 116.288) (end 136.906 117.094) (width 0.8) (layer F.Cu) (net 1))
 (segment (start 136.906 117.094) (end 142.748 117.094) (width 0.8) (layer F.Cu) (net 1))
 (segment (start 143.764 116.078) (end 143.764 114.989) (width 0.8) (layer F.Cu) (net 1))
 (segment (start 142.748 117.094) (end 143.764 116.078) (width 0.8) (layer F.Cu) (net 1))
 (segment (start 153.67 107.97) (end 151.11 105.41) (width 0.8) (layer F.Cu) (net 1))
 (segment (start 153.67 108.2405) (end 153.67 107.97) (width 0.8) (layer F.Cu) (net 1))
 (segment (start 155.48 105.95) (end 154.94 105.41) (width 0.8) (layer F.Cu) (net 16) (status 30))
 (segment (start 155.48 109.474) (end 155.48 105.95) (width 0.8) (layer F.Cu) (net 16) (status 30))
 (segment (start 153.7385 111.2155) (end 155.48 109.474) (width 0.8) (layer F.Cu) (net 16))
 (segment (start 153.67 111.2155) (end 153.7385 111.2155) (width 0.8) (layer F.Cu) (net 16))
 (segment (start 144.034 105.934) (end 143.51 105.41) (width 0.8) (layer F.Cu) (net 17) (status 30))
 (segment (start 144.034 109.474) (end 144.034 105.934) (width 0.8) (layer F.Cu) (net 17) (status 30))
 (segment (start 143.764 105.664) (end 143.51 105.41) (width 0.8) (layer F.Cu) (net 17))
 (segment (start 143.764 112.014) (end 143.764 105.664) (width 0.8) (layer F.Cu) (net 17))
 (segment (start 169.418 87.63) (end 172.72 87.63) (width 1.5) (layer B.Cu) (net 3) (status 20))
 (segment (start 151.11 115.61) (end 162.54 115.61) (width 1.5) (layer B.Cu) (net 3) (status 30))
 (segment (start 162.54 115.61) (end 165.06 115.61) (width 1.5) (layer B.Cu) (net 3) (status 10))
 (segment (start 165.06 115.61) (end 169.418 111.252) (width 1.5) (layer B.Cu) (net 3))
 (segment (start 169.164 89.662) (end 169.418 89.408) (width 1.5) (layer B.Cu) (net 3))
 (segment (start 166.37 89.662) (end 169.164 89.662) (width 1.5) (layer B.Cu) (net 3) (status 10))
 (segment (start 169.418 89.408) (end 169.418 87.63) (width 1.5) (layer B.Cu) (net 3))
 (segment (start 169.418 111.252) (end 169.418 89.408) (width 1.5) (layer B.Cu) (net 3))
 (segment (start 151.11 121.432) (end 153.162 119.38) (width 1.5) (layer F.Cu) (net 14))
 (segment (start 153.162 119.38) (end 165.1 119.38) (width 1.5) (layer F.Cu) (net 14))
 (segment (start 165.1 119.38) (end 168.91 115.57) (width 1.5) (layer F.Cu) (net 14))
 (segment (start 168.91 115.57) (end 168.91 105.41) (width 1.5) (layer F.Cu) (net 14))
 (segment (start 170.942 103.378) (end 173.228 103.378) (width 1.5) (layer F.Cu) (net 14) (status 20))
 (segment (start 168.91 105.41) (end 170.942 103.378) (width 1.5) (layer F.Cu) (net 14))
 (segment (start 151.11 121.432) (end 151.11 123.31) (width 1.5) (layer F.Cu) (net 14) (status 20))
 (segment (start 144.4 93.98) (end 144.78 94.36) (width 0.8) (layer F.Cu) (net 11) (status 30))
 (segment (start 139.7 93.98) (end 144.4 93.98) (width 0.8) (layer F.Cu) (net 11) (status 20))
 (segment (start 132.08 90.17) (end 133.35 90.17) (width 0.8) (layer F.Cu) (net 11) (status 10))
 (segment (start 139.7 93.98) (end 135.89 90.17) (width 0.8) (layer F.Cu) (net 11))
 (segment (start 134.62 90.17) (end 134.62 89.335) (width 1) (layer F.Cu) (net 11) (status 20))
 (segment (start 135.89 90.17) (end 134.62 90.17) (width 0.8) (layer F.Cu) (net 11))
 (segment (start 134.62 90.17) (end 132.08 90.17) (width 0.8) (layer F.Cu) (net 11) (status 20))
 (segment (start 135.73 96.36) (end 134.62 95.25) (width 0.8) (layer F.Cu) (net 10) (status 20))
 (segment (start 144.78 96.36) (end 135.73 96.36) (width 0.8) (layer F.Cu) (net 10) (status 10))
 (segment (start 134.62 95.25) (end 131.572 95.25) (width 0.8) (layer F.Cu) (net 10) (status 30))
 (segment (start 162.315 110) (end 162.56 110.245) (width 0.8) (layer F.Cu) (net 18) (status 30))
 (segment (start 160.02 110) (end 162.315 110) (width 0.8) (layer F.Cu) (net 18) (status 30))
 (segment (start 159.841 110.424) (end 160.02 110.245) (width 0.8) (layer F.Cu) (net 18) (status 30))
 (segment (start 157.48 110.424) (end 159.841 110.424) (width 0.8) (layer F.Cu) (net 18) (status 30))
 (segment (start 148.59 110) (end 148.59 110.49) (width 0.8) (layer F.Cu) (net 19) (status 30))
 (segment (start 148.59 110.49) (end 151.13 110.49) (width 0.8) (layer F.Cu) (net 19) (status 30))
 (segment (start 148.44 109.85) (end 148.59 110) (width 0.8) (layer F.Cu) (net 19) (status 30))
 (segment (start 148.157 110.424) (end 148.336 110.245) (width 1) (layer F.Cu) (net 19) (status 30))
 (segment (start 146.034 110.424) (end 148.157 110.424) (width 1) (layer F.Cu) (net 19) (status 30))
 (segment (start 162.56 108.195) (end 164.855 108.195) (width 0.8) (layer F.Cu) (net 6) (status 10))
 (segment (start 164.855 108.195) (end 164.855 103.895) (width 0.8) (layer B.Cu) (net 6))
 (via (at 164.855 108.195) (size 0.8) (drill 0.4) (layers F.Cu B.Cu) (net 6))
 (via (at 156.718 92.36) (size 0.8) (drill 0.4) (layers F.Cu B.Cu) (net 6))
 (segment (start 158.78 92.36) (end 156.718 92.36) (width 0.8) (layer F.Cu) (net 6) (status 10))
 (segment (start 163.322 102.362) (end 159.766 102.362) (width 0.8) (layer B.Cu) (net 6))
 (segment (start 164.855 103.895) (end 163.322 102.362) (width 0.8) (layer B.Cu) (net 6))
 (segment (start 156.718 99.314) (end 156.718 94.742) (width 0.8) (layer B.Cu) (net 6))
 (segment (start 159.766 102.362) (end 156.718 99.314) (width 0.8) (layer B.Cu) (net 6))
 (segment (start 156.718 94.742) (end 156.718 92.36) (width 0.8) (layer B.Cu) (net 6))
 (via (at 152.908 90.36) (size 0.8) (drill 0.4) (layers F.Cu B.Cu) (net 5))
 (segment (start 151.13 108.195) (end 148.336 105.401) (width 0.6) (layer F.Cu) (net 5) (status 10))
 (segment (start 148.336 105.401) (end 148.336 94.996) (width 0.6) (layer F.Cu) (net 5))
 (segment (start 148.336 94.996) (end 149.733 93.599) (width 0.6) (layer F.Cu) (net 5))
 (segment (start 149.733 93.599) (end 149.86 93.472) (width 0.6) (layer F.Cu) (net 5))
 (via (at 149.733 93.599) (size 0.8) (drill 0.4) (layers F.Cu B.Cu) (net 5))
 (segment (start 149.733 93.599) (end 152.908 90.424) (width 0.6) (layer B.Cu) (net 5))
 (segment (start 152.908 90.36) (end 158.78 90.36) (width 0.6) (layer F.Cu) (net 5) (status 20))
 (segment (start 141.478 83.82) (end 141.986 83.82) (width 0.8) (layer F.Cu) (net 13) (status 30))
 (segment (start 144.526 86.36) (end 144.78 86.36) (width 0.8) (layer F.Cu) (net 13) (status 30))
 (segment (start 142.24 83.82) (end 144.78 86.36) (width 0.8) (layer F.Cu) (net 13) (status 20))
 (segment (start 141.478 83.82) (end 142.24 83.82) (width 0.8) (layer F.Cu) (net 13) (status 10))
 (segment (start 140.97 88.41) (end 140.97 90.17) (width 0.8) (layer F.Cu) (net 12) (status 10))
 (segment (start 144.59 90.17) (end 144.78 90.36) (width 0.8) (layer F.Cu) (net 12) (status 30))
 (segment (start 140.97 90.17) (end 144.59 90.17) (width 0.8) (layer F.Cu) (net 12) (status 20))
 (segment (start 141.478 81.28) (end 142.494 81.28) (width 0.8) (layer F.Cu) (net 7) (status 10))
 (segment (start 142.494 81.28) (end 147.828 86.614) (width 0.8) (layer F.Cu) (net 7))
 (segment (start 147.828 86.614) (end 147.828 89.154) (width 0.8) (layer F.Cu) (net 7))
 (segment (start 153.034 94.36) (end 158.78 94.36) (width 0.8) (layer F.Cu) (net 7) (status 20))
 (segment (start 147.828 89.154) (end 153.034 94.36) (width 0.8) (layer F.Cu) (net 7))
 (segment (start 161.99 98.36) (end 162.56 97.79) (width 0.8) (layer F.Cu) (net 8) (status 20))
 (segment (start 158.78 98.36) (end 161.99 98.36) (width 0.8) (layer F.Cu) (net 8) (status 10))
 (segment (start 162.54 123.31) (end 166.25 123.31) (width 1.5) (layer B.Cu) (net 15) (status 10))
 (segment (start 173.228 116.332) (end 173.228 113.538) (width 1.5) (layer B.Cu) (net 15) (status 20))
 (segment (start 166.25 123.31) (end 173.228 116.332) (width 1.5) (layer B.Cu) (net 15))
 (segment (start 178.054 94.742) (end 176.022 92.71) (width 1.5) (layer B.Cu) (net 2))
 (segment (start 176.022 92.71) (end 173.228 92.71) (width 1.5) (layer B.Cu) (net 2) (status 20))
 (segment (start 178.054 106.934) (end 178.054 94.742) (width 1.5) (layer B.Cu) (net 2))
 (segment (start 176.53 108.458) (end 178.054 106.934) (width 1.5) (layer B.Cu) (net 2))
 (segment (start 173.228 108.458) (end 176.53 108.458) (width 1.5) (layer B.Cu) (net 2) (status 10))
 (segment (start 166.37 94.662) (end 169.244 94.662) (width 1.5) (layer F.Cu) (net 2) (status 10))
 (segment (start 171.196 92.71) (end 173.228 92.71) (width 1.5) (layer F.Cu) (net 2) (status 20))
 (segment (start 169.244 94.662) (end 171.196 92.71) (width 1.5) (layer F.Cu) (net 2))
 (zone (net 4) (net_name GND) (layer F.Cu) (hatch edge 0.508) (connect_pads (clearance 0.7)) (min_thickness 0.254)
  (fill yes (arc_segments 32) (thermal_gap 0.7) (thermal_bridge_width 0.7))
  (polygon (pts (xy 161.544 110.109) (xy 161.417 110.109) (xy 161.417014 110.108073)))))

